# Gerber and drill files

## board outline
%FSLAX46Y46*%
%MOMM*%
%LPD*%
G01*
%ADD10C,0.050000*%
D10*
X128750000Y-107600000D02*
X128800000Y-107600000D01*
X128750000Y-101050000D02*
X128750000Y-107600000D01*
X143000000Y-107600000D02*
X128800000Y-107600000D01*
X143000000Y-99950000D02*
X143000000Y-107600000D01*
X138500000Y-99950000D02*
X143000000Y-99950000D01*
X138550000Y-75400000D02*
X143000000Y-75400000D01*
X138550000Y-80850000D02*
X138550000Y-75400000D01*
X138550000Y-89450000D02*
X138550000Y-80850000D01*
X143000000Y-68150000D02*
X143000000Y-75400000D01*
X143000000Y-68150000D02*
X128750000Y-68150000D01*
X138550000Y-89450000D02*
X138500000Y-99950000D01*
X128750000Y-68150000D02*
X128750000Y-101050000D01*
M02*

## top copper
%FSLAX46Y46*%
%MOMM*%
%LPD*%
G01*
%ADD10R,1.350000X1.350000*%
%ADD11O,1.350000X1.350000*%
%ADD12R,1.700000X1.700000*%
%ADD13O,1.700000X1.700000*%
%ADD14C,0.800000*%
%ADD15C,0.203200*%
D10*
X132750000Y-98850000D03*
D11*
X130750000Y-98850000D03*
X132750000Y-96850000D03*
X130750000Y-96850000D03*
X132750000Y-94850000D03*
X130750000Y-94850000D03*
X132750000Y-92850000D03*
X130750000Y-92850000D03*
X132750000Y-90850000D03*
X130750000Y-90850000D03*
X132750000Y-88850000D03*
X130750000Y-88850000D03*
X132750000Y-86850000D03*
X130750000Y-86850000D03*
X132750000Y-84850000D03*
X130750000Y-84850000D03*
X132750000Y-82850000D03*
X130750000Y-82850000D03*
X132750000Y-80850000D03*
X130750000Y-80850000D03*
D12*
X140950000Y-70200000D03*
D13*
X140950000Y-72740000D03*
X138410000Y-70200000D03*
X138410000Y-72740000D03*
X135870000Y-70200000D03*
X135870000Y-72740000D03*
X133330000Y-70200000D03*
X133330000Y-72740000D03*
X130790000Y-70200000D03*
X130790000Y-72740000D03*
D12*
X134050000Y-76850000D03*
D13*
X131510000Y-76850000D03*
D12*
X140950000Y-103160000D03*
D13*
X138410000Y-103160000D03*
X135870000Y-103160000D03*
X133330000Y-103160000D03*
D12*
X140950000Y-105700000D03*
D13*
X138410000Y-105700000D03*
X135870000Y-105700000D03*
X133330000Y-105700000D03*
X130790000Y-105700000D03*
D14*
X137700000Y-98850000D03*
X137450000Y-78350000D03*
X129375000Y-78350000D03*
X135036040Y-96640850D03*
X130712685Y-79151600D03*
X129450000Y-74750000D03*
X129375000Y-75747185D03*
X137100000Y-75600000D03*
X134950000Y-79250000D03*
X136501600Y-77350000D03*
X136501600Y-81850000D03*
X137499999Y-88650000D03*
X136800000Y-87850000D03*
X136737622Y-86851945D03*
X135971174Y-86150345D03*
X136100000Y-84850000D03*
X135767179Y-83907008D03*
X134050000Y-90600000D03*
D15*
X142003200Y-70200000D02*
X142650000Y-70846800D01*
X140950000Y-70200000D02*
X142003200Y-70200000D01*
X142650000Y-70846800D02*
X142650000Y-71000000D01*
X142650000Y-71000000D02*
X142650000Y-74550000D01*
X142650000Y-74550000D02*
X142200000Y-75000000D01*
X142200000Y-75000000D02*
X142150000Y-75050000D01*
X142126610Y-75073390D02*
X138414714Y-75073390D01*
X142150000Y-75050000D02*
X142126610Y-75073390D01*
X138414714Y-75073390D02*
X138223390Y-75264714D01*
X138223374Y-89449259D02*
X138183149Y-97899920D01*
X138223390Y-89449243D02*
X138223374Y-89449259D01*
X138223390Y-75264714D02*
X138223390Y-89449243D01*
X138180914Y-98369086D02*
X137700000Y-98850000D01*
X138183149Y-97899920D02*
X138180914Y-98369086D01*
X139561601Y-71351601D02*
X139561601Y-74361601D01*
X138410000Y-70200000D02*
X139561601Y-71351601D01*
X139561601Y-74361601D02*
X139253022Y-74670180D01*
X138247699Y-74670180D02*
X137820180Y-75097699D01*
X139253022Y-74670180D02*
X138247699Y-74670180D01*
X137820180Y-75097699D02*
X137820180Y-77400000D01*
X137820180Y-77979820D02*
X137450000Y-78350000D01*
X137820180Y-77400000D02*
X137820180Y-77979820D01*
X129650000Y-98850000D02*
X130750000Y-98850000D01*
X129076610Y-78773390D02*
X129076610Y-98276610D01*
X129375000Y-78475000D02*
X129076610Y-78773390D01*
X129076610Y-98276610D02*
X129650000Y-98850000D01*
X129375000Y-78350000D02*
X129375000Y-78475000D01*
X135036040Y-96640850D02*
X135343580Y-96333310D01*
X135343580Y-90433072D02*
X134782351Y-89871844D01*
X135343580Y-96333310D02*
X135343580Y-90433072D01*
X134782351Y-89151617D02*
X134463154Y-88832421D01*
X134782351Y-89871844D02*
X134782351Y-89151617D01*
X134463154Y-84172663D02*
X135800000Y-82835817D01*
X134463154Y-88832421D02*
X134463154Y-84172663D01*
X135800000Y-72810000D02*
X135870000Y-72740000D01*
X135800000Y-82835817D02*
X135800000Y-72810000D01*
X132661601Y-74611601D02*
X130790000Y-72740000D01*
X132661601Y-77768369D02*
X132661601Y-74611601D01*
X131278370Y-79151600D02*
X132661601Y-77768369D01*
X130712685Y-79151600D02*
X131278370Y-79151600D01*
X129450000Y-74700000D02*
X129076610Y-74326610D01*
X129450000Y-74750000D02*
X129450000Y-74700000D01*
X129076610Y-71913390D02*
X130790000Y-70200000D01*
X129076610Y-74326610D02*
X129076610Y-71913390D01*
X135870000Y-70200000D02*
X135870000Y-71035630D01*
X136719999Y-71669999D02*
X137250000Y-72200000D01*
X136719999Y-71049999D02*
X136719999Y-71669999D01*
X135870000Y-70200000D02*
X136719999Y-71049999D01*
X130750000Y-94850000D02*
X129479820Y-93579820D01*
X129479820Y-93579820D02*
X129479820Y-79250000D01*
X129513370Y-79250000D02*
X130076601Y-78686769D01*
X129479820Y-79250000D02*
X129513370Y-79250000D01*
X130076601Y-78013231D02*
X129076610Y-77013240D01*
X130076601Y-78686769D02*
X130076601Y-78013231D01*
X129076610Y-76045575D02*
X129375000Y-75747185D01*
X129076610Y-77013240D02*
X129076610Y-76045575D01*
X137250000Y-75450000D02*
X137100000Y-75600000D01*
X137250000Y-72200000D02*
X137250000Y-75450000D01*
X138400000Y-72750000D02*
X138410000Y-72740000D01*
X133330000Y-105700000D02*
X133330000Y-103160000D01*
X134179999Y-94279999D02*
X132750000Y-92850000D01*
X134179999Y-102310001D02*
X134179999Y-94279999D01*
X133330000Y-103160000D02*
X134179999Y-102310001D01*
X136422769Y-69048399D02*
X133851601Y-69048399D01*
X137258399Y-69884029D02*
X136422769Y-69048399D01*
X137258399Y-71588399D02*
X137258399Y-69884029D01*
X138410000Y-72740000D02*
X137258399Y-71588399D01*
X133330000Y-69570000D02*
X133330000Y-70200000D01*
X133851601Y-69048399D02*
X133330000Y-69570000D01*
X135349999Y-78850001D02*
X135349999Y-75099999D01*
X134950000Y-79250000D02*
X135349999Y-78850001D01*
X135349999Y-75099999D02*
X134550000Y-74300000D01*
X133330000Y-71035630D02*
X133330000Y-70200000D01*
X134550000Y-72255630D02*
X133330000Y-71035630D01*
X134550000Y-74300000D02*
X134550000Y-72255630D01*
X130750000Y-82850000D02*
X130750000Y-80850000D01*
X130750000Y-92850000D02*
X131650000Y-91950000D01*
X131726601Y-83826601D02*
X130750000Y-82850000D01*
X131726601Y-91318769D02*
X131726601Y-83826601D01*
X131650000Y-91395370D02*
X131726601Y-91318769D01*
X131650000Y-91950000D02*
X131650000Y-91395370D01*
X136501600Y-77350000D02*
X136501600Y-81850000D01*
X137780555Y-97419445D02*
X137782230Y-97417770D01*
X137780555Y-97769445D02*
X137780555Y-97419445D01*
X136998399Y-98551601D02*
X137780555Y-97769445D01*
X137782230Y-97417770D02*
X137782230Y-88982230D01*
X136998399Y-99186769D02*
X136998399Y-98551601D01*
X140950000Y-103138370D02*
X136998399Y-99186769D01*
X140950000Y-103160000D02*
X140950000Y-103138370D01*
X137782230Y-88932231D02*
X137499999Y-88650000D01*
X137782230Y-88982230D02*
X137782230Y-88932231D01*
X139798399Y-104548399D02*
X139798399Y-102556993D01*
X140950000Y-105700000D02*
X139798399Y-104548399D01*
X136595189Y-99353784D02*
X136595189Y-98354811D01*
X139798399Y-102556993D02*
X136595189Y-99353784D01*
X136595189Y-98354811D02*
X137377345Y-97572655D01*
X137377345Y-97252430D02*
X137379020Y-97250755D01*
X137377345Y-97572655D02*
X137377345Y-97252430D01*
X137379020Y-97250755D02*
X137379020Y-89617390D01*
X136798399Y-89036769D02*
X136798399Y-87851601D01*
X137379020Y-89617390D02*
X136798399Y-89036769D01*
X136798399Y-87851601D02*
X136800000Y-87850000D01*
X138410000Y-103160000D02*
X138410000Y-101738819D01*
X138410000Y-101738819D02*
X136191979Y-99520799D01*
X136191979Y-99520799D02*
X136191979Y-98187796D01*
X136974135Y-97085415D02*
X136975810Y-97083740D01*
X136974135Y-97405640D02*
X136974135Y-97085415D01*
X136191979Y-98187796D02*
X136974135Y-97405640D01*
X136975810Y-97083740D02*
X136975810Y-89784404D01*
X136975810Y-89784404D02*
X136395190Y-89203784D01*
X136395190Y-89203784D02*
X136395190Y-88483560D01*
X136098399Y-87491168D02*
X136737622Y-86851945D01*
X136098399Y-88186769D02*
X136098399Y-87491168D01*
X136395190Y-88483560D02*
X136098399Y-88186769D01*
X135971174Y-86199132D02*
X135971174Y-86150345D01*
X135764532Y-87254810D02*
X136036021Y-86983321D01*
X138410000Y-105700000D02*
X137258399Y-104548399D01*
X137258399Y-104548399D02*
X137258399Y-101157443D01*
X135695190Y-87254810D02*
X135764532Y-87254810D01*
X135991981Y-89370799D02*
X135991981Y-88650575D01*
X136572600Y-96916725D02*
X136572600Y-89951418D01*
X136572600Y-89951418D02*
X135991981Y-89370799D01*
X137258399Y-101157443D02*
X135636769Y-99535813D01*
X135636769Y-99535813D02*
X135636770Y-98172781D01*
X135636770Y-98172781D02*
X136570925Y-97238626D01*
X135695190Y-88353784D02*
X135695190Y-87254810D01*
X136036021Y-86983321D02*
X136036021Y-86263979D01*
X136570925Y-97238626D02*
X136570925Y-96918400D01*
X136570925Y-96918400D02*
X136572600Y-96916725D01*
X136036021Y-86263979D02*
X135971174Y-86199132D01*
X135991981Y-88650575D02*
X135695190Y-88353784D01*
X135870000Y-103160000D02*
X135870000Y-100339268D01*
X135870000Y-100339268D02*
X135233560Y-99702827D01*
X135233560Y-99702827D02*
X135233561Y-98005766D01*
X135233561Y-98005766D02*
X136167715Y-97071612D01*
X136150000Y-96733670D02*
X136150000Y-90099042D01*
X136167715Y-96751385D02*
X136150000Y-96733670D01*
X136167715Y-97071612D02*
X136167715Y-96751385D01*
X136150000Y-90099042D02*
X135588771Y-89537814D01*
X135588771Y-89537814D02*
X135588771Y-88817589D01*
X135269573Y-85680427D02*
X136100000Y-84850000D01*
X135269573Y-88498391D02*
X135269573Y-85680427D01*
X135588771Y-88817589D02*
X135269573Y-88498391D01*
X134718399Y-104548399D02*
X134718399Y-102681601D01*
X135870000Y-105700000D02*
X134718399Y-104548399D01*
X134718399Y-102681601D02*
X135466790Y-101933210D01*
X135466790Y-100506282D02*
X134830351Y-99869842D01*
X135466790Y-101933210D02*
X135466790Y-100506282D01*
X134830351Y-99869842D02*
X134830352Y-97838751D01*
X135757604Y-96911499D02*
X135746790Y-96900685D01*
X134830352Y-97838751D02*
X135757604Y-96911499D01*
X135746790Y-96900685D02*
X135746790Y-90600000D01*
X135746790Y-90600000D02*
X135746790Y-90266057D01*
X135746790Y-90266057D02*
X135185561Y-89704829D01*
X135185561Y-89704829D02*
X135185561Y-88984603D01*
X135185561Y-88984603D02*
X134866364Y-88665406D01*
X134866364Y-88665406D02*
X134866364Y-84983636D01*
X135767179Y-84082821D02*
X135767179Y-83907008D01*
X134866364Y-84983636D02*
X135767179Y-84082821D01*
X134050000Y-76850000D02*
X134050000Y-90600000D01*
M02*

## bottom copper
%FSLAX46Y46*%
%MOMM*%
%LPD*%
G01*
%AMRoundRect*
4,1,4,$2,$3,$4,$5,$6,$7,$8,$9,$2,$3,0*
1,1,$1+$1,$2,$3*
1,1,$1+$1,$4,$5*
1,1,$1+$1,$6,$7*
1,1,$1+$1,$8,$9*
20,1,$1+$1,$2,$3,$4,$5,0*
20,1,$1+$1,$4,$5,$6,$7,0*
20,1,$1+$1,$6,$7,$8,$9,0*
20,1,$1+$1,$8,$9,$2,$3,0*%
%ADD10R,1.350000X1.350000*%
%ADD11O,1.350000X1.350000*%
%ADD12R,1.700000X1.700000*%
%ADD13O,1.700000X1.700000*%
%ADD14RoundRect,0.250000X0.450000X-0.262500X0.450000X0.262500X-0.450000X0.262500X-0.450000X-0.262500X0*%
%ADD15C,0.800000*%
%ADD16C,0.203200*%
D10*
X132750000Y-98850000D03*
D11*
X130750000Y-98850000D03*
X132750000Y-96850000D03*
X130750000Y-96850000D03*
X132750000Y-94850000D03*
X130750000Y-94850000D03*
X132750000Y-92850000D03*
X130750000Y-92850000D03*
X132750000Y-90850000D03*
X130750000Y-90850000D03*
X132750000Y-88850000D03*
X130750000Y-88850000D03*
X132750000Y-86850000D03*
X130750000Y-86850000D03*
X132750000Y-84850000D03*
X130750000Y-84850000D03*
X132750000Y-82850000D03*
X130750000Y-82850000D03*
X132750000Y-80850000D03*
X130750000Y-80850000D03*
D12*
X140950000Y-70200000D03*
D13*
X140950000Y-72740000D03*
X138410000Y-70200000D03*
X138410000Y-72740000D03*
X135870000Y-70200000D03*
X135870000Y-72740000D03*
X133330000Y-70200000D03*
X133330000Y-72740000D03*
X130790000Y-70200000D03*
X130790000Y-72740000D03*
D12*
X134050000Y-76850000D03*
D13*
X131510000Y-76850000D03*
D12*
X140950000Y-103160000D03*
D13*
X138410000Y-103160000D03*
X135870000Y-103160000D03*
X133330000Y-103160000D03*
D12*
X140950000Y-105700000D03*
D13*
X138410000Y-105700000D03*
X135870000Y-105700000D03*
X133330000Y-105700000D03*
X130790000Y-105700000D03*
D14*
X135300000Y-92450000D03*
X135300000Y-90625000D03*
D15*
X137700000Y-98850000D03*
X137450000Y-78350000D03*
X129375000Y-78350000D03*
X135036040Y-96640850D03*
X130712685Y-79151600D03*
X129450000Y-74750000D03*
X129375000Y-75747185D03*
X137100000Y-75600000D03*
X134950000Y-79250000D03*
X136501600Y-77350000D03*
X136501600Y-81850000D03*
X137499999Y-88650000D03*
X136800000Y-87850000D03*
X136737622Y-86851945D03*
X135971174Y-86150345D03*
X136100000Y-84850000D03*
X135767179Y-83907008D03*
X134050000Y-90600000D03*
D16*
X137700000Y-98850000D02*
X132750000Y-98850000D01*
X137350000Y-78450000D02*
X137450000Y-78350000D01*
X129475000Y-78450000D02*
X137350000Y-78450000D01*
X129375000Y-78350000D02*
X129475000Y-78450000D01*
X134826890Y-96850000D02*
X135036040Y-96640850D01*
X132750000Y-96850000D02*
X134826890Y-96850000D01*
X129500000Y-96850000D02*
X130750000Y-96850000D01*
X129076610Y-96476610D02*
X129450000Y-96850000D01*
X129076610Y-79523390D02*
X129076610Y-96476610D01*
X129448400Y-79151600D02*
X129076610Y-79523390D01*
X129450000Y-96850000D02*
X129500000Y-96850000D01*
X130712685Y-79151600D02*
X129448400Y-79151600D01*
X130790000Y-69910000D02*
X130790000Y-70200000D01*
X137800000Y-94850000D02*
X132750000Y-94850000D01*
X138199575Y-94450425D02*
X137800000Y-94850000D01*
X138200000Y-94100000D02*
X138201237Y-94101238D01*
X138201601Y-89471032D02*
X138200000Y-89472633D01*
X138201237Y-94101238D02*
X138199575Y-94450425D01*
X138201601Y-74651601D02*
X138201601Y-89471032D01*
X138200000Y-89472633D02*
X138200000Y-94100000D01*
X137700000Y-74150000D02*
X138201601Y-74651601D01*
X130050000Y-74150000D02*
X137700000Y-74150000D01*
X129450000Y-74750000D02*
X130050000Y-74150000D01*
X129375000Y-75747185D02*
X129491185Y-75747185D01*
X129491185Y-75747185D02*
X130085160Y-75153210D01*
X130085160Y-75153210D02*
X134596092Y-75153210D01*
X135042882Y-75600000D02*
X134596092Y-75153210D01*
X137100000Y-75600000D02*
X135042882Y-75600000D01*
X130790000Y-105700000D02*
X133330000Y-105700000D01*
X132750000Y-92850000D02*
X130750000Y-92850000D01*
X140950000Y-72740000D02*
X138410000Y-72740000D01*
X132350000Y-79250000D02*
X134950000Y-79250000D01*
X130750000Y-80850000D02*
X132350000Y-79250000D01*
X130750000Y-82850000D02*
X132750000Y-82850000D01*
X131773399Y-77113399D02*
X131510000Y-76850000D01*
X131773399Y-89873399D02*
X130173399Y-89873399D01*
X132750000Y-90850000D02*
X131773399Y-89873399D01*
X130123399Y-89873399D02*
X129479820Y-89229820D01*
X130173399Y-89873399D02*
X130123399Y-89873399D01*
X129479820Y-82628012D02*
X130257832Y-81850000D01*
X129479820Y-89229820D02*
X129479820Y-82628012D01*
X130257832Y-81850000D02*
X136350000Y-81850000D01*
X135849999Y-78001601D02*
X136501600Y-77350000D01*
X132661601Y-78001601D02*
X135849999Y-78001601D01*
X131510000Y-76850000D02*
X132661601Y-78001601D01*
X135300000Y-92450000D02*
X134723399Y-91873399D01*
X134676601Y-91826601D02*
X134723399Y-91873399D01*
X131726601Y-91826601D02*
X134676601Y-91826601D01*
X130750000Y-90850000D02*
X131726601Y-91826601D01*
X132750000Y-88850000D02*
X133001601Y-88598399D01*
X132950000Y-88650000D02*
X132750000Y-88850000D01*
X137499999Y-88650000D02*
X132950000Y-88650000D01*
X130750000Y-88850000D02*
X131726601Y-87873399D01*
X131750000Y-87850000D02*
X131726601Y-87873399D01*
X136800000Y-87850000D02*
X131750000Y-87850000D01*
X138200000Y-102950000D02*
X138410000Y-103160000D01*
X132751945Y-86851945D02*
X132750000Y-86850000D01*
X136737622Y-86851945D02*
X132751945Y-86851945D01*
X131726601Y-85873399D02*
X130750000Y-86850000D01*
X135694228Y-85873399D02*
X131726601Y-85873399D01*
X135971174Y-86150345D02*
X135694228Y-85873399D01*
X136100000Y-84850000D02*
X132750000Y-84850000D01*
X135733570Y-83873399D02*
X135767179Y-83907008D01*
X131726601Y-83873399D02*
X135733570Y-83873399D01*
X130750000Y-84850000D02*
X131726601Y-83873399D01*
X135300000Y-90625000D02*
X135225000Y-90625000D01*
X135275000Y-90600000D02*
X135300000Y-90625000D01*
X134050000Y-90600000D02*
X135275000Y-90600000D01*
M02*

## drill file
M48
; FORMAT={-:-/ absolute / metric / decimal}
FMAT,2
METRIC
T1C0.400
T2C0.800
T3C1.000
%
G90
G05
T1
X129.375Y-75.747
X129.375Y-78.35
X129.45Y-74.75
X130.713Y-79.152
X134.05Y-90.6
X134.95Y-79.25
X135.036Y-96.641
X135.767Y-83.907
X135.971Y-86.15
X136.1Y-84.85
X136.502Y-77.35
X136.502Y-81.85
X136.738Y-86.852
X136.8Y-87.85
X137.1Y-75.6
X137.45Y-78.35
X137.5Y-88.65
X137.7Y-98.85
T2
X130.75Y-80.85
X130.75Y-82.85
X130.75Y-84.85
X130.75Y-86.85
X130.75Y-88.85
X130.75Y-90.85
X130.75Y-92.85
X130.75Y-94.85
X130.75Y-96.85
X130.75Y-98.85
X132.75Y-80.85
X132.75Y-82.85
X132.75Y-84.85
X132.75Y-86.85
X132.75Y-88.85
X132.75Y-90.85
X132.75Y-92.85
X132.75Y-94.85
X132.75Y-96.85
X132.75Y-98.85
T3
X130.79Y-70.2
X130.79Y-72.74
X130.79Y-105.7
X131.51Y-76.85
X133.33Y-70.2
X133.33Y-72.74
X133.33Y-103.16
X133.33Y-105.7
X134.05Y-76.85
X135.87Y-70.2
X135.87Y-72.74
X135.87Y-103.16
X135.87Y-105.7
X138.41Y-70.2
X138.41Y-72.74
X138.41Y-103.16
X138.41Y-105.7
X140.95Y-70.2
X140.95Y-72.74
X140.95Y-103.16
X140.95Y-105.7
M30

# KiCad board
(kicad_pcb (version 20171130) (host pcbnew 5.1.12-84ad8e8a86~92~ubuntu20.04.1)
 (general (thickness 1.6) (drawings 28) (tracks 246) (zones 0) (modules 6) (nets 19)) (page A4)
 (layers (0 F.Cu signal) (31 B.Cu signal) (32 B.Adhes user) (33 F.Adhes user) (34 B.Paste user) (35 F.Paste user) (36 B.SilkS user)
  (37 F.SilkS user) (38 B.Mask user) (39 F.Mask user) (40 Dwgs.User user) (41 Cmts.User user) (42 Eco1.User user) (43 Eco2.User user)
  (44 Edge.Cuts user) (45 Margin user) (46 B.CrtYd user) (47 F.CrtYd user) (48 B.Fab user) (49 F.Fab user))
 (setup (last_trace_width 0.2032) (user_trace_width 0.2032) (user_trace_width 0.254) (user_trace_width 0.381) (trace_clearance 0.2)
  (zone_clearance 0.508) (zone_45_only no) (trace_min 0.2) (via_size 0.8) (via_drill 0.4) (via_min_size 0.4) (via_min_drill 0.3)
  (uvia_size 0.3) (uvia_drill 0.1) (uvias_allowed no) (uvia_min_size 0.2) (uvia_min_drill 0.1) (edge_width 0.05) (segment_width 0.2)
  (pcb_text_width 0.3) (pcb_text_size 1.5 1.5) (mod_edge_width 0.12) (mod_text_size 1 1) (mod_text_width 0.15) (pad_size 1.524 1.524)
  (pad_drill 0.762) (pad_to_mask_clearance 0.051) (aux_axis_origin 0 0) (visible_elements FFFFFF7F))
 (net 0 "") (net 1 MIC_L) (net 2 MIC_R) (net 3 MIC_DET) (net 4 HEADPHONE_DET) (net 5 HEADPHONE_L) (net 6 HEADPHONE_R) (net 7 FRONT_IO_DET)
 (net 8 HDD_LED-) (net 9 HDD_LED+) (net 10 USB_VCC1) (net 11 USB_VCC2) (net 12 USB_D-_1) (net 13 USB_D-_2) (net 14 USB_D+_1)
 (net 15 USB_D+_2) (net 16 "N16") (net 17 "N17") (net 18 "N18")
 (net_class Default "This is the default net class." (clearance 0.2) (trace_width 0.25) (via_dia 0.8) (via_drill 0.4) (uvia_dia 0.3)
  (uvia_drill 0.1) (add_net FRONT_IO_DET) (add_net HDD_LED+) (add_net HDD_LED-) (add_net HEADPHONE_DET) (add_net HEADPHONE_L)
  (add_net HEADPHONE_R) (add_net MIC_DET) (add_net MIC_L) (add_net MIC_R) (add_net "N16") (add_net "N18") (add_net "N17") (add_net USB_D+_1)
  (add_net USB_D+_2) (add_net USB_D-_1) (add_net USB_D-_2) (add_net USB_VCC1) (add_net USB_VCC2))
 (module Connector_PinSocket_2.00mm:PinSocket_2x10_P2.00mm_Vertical (layer B.Cu) (at 132.75 98.85)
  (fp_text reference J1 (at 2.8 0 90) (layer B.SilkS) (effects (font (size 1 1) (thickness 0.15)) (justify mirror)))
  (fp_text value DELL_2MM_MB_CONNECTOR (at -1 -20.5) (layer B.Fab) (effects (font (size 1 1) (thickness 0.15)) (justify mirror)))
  (pad 1 thru_hole rect (at 0 0) (size 1.35 1.35) (drill 0.8) (layers *.Cu *.Mask) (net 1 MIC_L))
  (pad 2 thru_hole oval (at -2 0) (size 1.35 1.35) (drill 0.8) (layers *.Cu *.Mask) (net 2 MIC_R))
  (pad 3 thru_hole oval (at 0 -2) (size 1.35 1.35) (drill 0.8) (layers *.Cu *.Mask) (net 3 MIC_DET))
  (pad 4 thru_hole oval (at -2 -2) (size 1.35 1.35) (drill 0.8) (layers *.Cu *.Mask) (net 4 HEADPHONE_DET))
  (pad 5 thru_hole oval (at 0 -4) (size 1.35 1.35) (drill 0.8) (layers *.Cu *.Mask) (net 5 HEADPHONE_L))
  (pad 6 thru_hole oval (at -2 -4) (size 1.35 1.35) (drill 0.8) (layers *.Cu *.Mask) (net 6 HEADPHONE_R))
  (pad 7 thru_hole oval (at 0 -6) (size 1.35 1.35) (drill 0.8) (layers *.Cu *.Mask) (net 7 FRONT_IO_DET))
  (pad 8 thru_hole oval (at -2 -6) (size 1.35 1.35) (drill 0.8) (layers *.Cu *.Mask) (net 7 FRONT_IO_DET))
  (pad 9 thru_hole oval (at 0 -8) (size 1.35 1.35) (drill 0.8) (layers *.Cu *.Mask) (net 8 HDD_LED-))
  (pad 10 thru_hole oval (at -2 -8) (size 1.35 1.35) (drill 0.8) (layers *.Cu *.Mask) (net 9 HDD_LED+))
  (pad 11 thru_hole oval (at 0 -10) (size 1.35 1.35) (drill 0.8) (layers *.Cu *.Mask) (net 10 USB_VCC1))
  (pad 12 thru_hole oval (at -2 -10) (size 1.35 1.35) (drill 0.8) (layers *.Cu *.Mask) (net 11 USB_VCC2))
  (pad 13 thru_hole oval (at 0 -12) (size 1.35 1.35) (drill 0.8) (layers *.Cu *.Mask) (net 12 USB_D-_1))
  (pad 14 thru_hole oval (at -2 -12) (size 1.35 1.35) (drill 0.8) (layers *.Cu *.Mask) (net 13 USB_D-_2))
  (pad 15 thru_hole oval (at 0 -14) (size 1.35 1.35) (drill 0.8) (layers *.Cu *.Mask) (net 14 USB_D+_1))
  (pad 16 thru_hole oval (at -2 -14) (size 1.35 1.35) (drill 0.8) (layers *.Cu *.Mask) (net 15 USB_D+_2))
  (pad 17 thru_hole oval (at 0 -16) (size 1.35 1.35) (drill 0.8) (layers *.Cu *.Mask) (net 7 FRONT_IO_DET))
  (pad 18 thru_hole oval (at -2 -16) (size 1.35 1.35) (drill 0.8) (layers *.Cu *.Mask) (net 7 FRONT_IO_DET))
  (pad 19 thru_hole oval (at 0 -18) (size 1.35 1.35) (drill 0.8) (layers *.Cu *.Mask) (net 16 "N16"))
  (pad 20 thru_hole oval (at -2 -18) (size 1.35 1.35) (drill 0.8) (layers *.Cu *.Mask) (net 7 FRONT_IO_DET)))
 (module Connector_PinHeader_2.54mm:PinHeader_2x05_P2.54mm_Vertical (layer F.Cu) (at 140.95 70.2 270)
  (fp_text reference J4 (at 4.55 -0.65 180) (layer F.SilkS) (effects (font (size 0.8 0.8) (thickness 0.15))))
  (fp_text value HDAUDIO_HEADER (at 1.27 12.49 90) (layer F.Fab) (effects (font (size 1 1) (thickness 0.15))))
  (pad 1 thru_hole rect (at 0 0 270) (size 1.7 1.7) (drill 1) (layers *.Cu *.Mask) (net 1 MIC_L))
  (pad 2 thru_hole oval (at 2.54 0 270) (size 1.7 1.7) (drill 1) (layers *.Cu *.Mask) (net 7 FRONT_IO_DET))
  (pad 3 thru_hole oval (at 0 2.54 270) (size 1.7 1.7) (drill 1) (layers *.Cu *.Mask) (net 2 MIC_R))
  (pad 4 thru_hole oval (at 2.54 2.54 270) (size 1.7 1.7) (drill 1) (layers *.Cu *.Mask) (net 7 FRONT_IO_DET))
  (pad 5 thru_hole oval (at 0 5.08 270) (size 1.7 1.7) (drill 1) (layers *.Cu *.Mask) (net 6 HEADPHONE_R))
  (pad 6 thru_hole oval (at 2.54 5.08 270) (size 1.7 1.7) (drill 1) (layers *.Cu *.Mask) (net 3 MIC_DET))
  (pad 7 thru_hole oval (at 0 7.62 270) (size 1.7 1.7) (drill 1) (layers *.Cu *.Mask) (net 7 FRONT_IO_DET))
  (pad 8 thru_hole oval (at 2.54 7.62 270) (size 1.7 1.7) (drill 1) (layers *.Cu *.Mask) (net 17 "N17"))
  (pad 9 thru_hole oval (at 0 10.16 270) (size 1.7 1.7) (drill 1) (layers *.Cu *.Mask) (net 5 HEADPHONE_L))
  (pad 10 thru_hole oval (at 2.54 10.16 270) (size 1.7 1.7) (drill 1) (layers *.Cu *.Mask) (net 4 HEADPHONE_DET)))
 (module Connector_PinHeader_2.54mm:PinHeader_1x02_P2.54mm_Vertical (layer F.Cu) (at 134.05 76.85 270)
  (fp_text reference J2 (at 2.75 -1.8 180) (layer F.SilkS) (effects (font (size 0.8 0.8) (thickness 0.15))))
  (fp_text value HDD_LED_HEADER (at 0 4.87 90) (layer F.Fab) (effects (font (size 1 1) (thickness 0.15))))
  (pad 1 thru_hole rect (at 0 0 270) (size 1.7 1.7) (drill 1) (layers *.Cu *.Mask) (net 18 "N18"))
  (pad 2 thru_hole oval (at 0 2.54 270) (size 1.7 1.7) (drill 1) (layers *.Cu *.Mask) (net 8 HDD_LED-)))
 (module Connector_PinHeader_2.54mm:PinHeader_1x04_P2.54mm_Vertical (layer F.Cu) (at 140.95 103.16 270)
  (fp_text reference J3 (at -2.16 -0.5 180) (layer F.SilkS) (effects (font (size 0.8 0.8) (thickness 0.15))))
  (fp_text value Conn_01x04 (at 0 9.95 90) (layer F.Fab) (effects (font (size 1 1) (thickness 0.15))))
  (pad 1 thru_hole rect (at 0 0 270) (size 1.7 1.7) (drill 1) (layers *.Cu *.Mask) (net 10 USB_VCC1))
  (pad 2 thru_hole oval (at 0 2.54 270) (size 1.7 1.7) (drill 1) (layers *.Cu *.Mask) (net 12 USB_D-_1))
  (pad 3 thru_hole oval (at 0 5.08 270) (size 1.7 1.7) (drill 1) (layers *.Cu *.Mask) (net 14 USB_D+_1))
  (pad 4 thru_hole oval (at 0 7.62 270) (size 1.7 1.7) (drill 1) (layers *.Cu *.Mask) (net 7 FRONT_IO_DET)))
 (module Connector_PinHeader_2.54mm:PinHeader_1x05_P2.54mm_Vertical (layer F.Cu) (at 140.95 105.7 270)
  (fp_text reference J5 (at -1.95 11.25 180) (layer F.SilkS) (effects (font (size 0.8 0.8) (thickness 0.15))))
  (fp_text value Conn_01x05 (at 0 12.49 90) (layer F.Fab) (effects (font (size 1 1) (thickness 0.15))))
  (pad 1 thru_hole rect (at 0 0 270) (size 1.7 1.7) (drill 1) (layers *.Cu *.Mask) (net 11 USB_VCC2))
  (pad 2 thru_hole oval (at 0 2.54 270) (size 1.7 1.7) (drill 1) (layers *.Cu *.Mask) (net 13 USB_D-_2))
  (pad 3 thru_hole oval (at 0 5.08 270) (size 1.7 1.7) (drill 1) (layers *.Cu *.Mask) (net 15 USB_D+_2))
  (pad 4 thru_hole oval (at 0 7.62 270) (size 1.7 1.7) (drill 1) (layers *.Cu *.Mask) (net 7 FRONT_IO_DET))
  (pad 5 thru_hole oval (at 0 10.16 270) (size 1.7 1.7) (drill 1) (layers *.Cu *.Mask) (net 7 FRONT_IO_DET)))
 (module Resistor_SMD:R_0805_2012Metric (layer B.Cu) (at 135.3 91.5375 90)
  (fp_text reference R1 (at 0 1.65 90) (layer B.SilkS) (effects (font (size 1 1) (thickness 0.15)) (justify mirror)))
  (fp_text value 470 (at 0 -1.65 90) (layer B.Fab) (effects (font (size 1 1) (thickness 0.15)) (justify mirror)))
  (pad 1 smd roundrect (at -0.9125 0 90) (size 1.025 1.4) (layers B.Cu B.Paste B.Mask) (roundrect_rratio 0.243902) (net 9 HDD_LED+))
  (pad 2 smd roundrect (at 0.9125 0 90) (size 1.025 1.4) (layers B.Cu B.Paste B.Mask) (roundrect_rratio 0.243902) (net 18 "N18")))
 (gr_line (start 128.75 107.6) (end 128.8 107.6) (layer Edge.Cuts) (width 0.05))
 (gr_line (start 128.75 101.05) (end 128.75 107.6) (layer Edge.Cuts) (width 0.05))
 (gr_line (start 143 107.6) (end 128.8 107.6) (layer Edge.Cuts) (width 0.05))
 (gr_line (start 143 99.95) (end 143 107.6) (layer Edge.Cuts) (width 0.05))
 (gr_line (start 138.5 99.95) (end 143 99.95) (layer Edge.Cuts) (width 0.05))
 (gr_line (start 138.55 75.4) (end 143 75.4) (layer Edge.Cuts) (width 0.05))
 (gr_line (start 138.55 80.85) (end 138.55 75.4) (layer Edge.Cuts) (width 0.05))
 (gr_line (start 138.55 89.45) (end 138.55 80.85) (layer Edge.Cuts) (width 0.05))
 (gr_line (start 143 68.15) (end 143 75.4) (layer Edge.Cuts) (width 0.05))
 (gr_line (start 143 68.15) (end 128.75 68.15) (layer Edge.Cuts) (width 0.05))
 (gr_line (start 138.55 89.45) (end 138.5 99.95) (layer Edge.Cuts) (width 0.05))
 (gr_line (start 128.75 68.15) (end 128.75 101.05) (layer Edge.Cuts) (width 0.05))
 (segment (start 142.0032 70.2) (end 142.65 70.8468) (width 0.2032) (layer F.Cu) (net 1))
 (segment (start 140.95 70.2) (end 142.0032 70.2) (width 0.2032) (layer F.Cu) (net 1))
 (segment (start 142.65 70.8468) (end 142.65 71) (width 0.2032) (layer F.Cu) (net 1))
 (segment (start 142.65 71) (end 142.65 74.55) (width 0.2032) (layer F.Cu) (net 1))
 (segment (start 142.65 74.55) (end 142.2 75) (width 0.2032) (layer F.Cu) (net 1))
 (segment (start 142.2 75) (end 142.15 75.05) (width 0.2032) (layer F.Cu) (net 1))
 (segment (start 142.12661 75.07339) (end 138.414714 75.07339) (width 0.2032) (layer F.Cu) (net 1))
 (segment (start 142.15 75.05) (end 142.12661 75.07339) (width 0.2032) (layer F.Cu) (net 1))
 (segment (start 138.414714 75.07339) (end 138.22339 75.264714) (width 0.2032) (layer F.Cu) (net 1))
 (segment (start 138.223374 89.449259) (end 138.183149 97.89992) (width 0.2032) (layer F.Cu) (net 1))
 (segment (start 138.22339 89.449243) (end 138.223374 89.449259) (width 0.2032) (layer F.Cu) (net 1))
 (segment (start 138.22339 75.264714) (end 138.22339 89.449243) (width 0.2032) (layer F.Cu) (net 1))
 (via (at 137.7 98.85) (size 0.8) (drill 0.4) (layers F.Cu B.Cu) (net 1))
 (segment (start 138.180914 98.369086) (end 137.7 98.85) (width 0.2032) (layer F.Cu) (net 1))
 (segment (start 138.183149 97.89992) (end 138.180914 98.369086) (width 0.2032) (layer F.Cu) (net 1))
 (segment (start 137.7 98.85) (end 132.75 98.85) (width 0.2032) (layer B.Cu) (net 1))
 (segment (start 139.561601 71.351601) (end 139.561601 74.361601) (width 0.2032) (layer F.Cu) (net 2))
 (segment (start 138.41 70.2) (end 139.561601 71.351601) (width 0.2032) (layer F.Cu) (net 2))
 (segment (start 139.561601 74.361601) (end 139.253022 74.67018) (width 0.2032) (layer F.Cu) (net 2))
 (segment (start 138.247699 74.67018) (end 137.82018 75.097699) (width 0.2032) (layer F.Cu) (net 2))
 (segment (start 139.253022 74.67018) (end 138.247699 74.67018) (width 0.2032) (layer F.Cu) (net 2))
 (segment (start 137.82018 75.097699) (end 137.82018 77.4) (width 0.2032) (layer F.Cu) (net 2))
 (via (at 137.45 78.35) (size 0.8) (drill 0.4) (layers F.Cu B.Cu) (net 2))
 (segment (start 137.82018 77.97982) (end 137.45 78.35) (width 0.2032) (layer F.Cu) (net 2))
 (segment (start 137.82018 77.4) (end 137.82018 77.97982) (width 0.2032) (layer F.Cu) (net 2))
 (via (at 129.375 78.35) (size 0.8) (drill 0.4) (layers F.Cu B.Cu) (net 2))
 (segment (start 129.65 98.85) (end 130.75 98.85) (width 0.2032) (layer F.Cu) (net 2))
 (segment (start 129.07661 78.77339) (end 129.07661 98.27661) (width 0.2032) (layer F.Cu) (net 2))
 (segment (start 129.375 78.475) (end 129.07661 78.77339) (width 0.2032) (layer F.Cu) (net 2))
 (segment (start 129.07661 98.27661) (end 129.65 98.85) (width 0.2032) (layer F.Cu) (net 2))
 (segment (start 129.375 78.35) (end 129.375 78.475) (width 0.2032) (layer F.Cu) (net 2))
 (segment (start 137.35 78.45) (end 137.45 78.35) (width 0.2032) (layer B.Cu) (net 2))
 (segment (start 129.475 78.45) (end 137.35 78.45) (width 0.2032) (layer B.Cu) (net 2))
 (segment (start 129.375 78.35) (end 129.475 78.45) (width 0.2032) (layer B.Cu) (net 2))
 (via (at 135.03604 96.64085) (size 0.8) (drill 0.4) (layers F.Cu B.Cu) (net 3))
 (segment (start 134.82689 96.85) (end 135.03604 96.64085) (width 0.2032) (layer B.Cu) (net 3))
 (segment (start 132.75 96.85) (end 134.82689 96.85) (width 0.2032) (layer B.Cu) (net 3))
 (segment (start 135.03604 96.64085) (end 135.34358 96.33331) (width 0.2032) (layer F.Cu) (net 3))
 (segment (start 135.34358 90.433072) (end 134.782351 89.871844) (width 0.2032) (layer F.Cu) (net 3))
 (segment (start 135.34358 96.33331) (end 135.34358 90.433072) (width 0.2032) (layer F.Cu) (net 3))
 (segment (start 134.782351 89.151617) (end 134.463154 88.832421) (width 0.2032) (layer F.Cu) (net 3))
 (segment (start 134.782351 89.871844) (end 134.782351 89.151617) (width 0.2032) (layer F.Cu) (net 3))
 (segment (start 134.463154 84.172663) (end 135.8 82.835817) (width 0.2032) (layer F.Cu) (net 3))
 (segment (start 134.463154 88.832421) (end 134.463154 84.172663) (width 0.2032) (layer F.Cu) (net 3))
 (segment (start 135.8 72.81) (end 135.87 72.74) (width 0.2032) (layer F.Cu) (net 3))
 (segment (start 135.8 82.835817) (end 135.8 72.81) (width 0.2032) (layer F.Cu) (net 3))
 (via (at 130.712685 79.1516) (size 0.8) (drill 0.4) (layers F.Cu B.Cu) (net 4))
 (segment (start 132.661601 74.611601) (end 130.79 72.74) (width 0.2032) (layer F.Cu) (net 4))
 (segment (start 132.661601 77.768369) (end 132.661601 74.611601) (width 0.2032) (layer F.Cu) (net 4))
 (segment (start 131.27837 79.1516) (end 132.661601 77.768369) (width 0.2032) (layer F.Cu) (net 4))
 (segment (start 130.712685 79.1516) (end 131.27837 79.1516) (width 0.2032) (layer F.Cu) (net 4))
 (segment (start 129.5 96.85) (end 130.75 96.85) (width 0.2032) (layer B.Cu) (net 4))
 (segment (start 129.07661 96.47661) (end 129.45 96.85) (width 0.2032) (layer B.Cu) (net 4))
 (segment (start 129.07661 79.52339) (end 129.07661 96.47661) (width 0.2032) (layer B.Cu) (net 4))
 (segment (start 129.4484 79.1516) (end 129.07661 79.52339) (width 0.2032) (layer B.Cu) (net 4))
 (segment (start 129.45 96.85) (end 129.5 96.85) (width 0.2032) (layer B.Cu) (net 4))
 (segment (start 130.712685 79.1516) (end 129.4484 79.1516) (width 0.2032) (layer B.Cu) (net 4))
 (segment (start 130.79 69.91) (end 130.79 70.2) (width 0.2032) (layer B.Cu) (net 5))
 (via (at 129.45 74.75) (size 0.8) (drill 0.4) (layers F.Cu B.Cu) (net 5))
 (segment (start 129.45 74.7) (end 129.07661 74.32661) (width 0.2032) (layer F.Cu) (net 5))
 (segment (start 129.45 74.75) (end 129.45 74.7) (width 0.2032) (layer F.Cu) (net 5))
 (segment (start 129.07661 71.91339) (end 130.79 70.2) (width 0.2032) (layer F.Cu) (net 5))
 (segment (start 129.07661 74.32661) (end 129.07661 71.91339) (width 0.2032) (layer F.Cu) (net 5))
 (segment (start 137.8 94.85) (end 132.75 94.85) (width 0.2032) (layer B.Cu) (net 5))
 (segment (start 138.199575 94.450425) (end 137.8 94.85) (width 0.2032) (layer B.Cu) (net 5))
 (segment (start 138.2 94.1) (end 138.201237 94.101238) (width 0.2032) (layer B.Cu) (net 5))
 (segment (start 138.201601 89.471032) (end 138.2 89.472633) (width 0.2032) (layer B.Cu) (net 5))
 (segment (start 138.201237 94.101238) (end 138.199575 94.450425) (width 0.2032) (layer B.Cu) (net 5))
 (segment (start 138.201601 74.651601) (end 138.201601 89.471032) (width 0.2032) (layer B.Cu) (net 5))
 (segment (start 138.2 89.472633) (end 138.2 94.1) (width 0.2032) (layer B.Cu) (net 5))
 (segment (start 137.7 74.15) (end 138.201601 74.651601) (width 0.2032) (layer B.Cu) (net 5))
 (segment (start 130.05 74.15) (end 137.7 74.15) (width 0.2032) (layer B.Cu) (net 5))
 (segment (start 129.45 74.75) (end 130.05 74.15) (width 0.2032) (layer B.Cu) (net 5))
 (segment (start 135.87 70.2) (end 135.87 71.03563) (width 0.2032) (layer F.Cu) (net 6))
 (segment (start 136.719999 71.669999) (end 137.25 72.2) (width 0.2032) (layer F.Cu) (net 6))
 (segment (start 136.719999 71.049999) (end 136.719999 71.669999) (width 0.2032) (layer F.Cu) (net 6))
 (segment (start 135.87 70.2) (end 136.719999 71.049999) (width 0.2032) (layer F.Cu) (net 6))
 (segment (start 130.75 94.85) (end 129.47982 93.57982) (width 0.2032) (layer F.Cu) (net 6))
 (segment (start 129.47982 93.57982) (end 129.47982 79.25) (width 0.2032) (layer F.Cu) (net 6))
 (segment (start 129.51337 79.25) (end 130.076601 78.686769) (width 0.2032) (layer F.Cu) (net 6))
 (segment (start 129.47982 79.25) (end 129.51337 79.25) (width 0.2032) (layer F.Cu) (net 6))
 (segment (start 130.076601 78.013231) (end 129.07661 77.01324) (width 0.2032) (layer F.Cu) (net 6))
 (segment (start 130.076601 78.686769) (end 130.076601 78.013231) (width 0.2032) (layer F.Cu) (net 6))
 (via (at 129.375 75.747185) (size 0.8) (drill 0.4) (layers F.Cu B.Cu) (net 6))
 (segment (start 129.07661 76.045575) (end 129.375 75.747185) (width 0.2032) (layer F.Cu) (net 6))
 (segment (start 129.07661 77.01324) (end 129.07661 76.045575) (width 0.2032) (layer F.Cu) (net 6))
 (segment (start 129.375 75.747185) (end 129.491185 75.747185) (width 0.2032) (layer B.Cu) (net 6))
 (segment (start 129.491185 75.747185) (end 130.08516 75.15321) (width 0.2032) (layer B.Cu) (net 6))
 (segment (start 130.08516 75.15321) (end 134.596092 75.15321) (width 0.2032) (layer B.Cu) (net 6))
 (via (at 137.1 75.6) (size 0.8) (drill 0.4) (layers F.Cu B.Cu) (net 6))
 (segment (start 137.25 75.45) (end 137.1 75.6) (width 0.2032) (layer F.Cu) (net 6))
 (segment (start 137.25 72.2) (end 137.25 75.45) (width 0.2032) (layer F.Cu) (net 6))
 (segment (start 135.042882 75.6) (end 134.596092 75.15321) (width 0.2032) (layer B.Cu) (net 6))
 (segment (start 137.1 75.6) (end 135.042882 75.6) (width 0.2032) (layer B.Cu) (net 6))
 (segment (start 138.4 72.75) (end 138.41 72.74) (width 0.2032) (layer F.Cu) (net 7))
 (segment (start 130.79 105.7) (end 133.33 105.7) (width 0.2032) (layer B.Cu) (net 7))
 (segment (start 133.33 105.7) (end 133.33 103.16) (width 0.2032) (layer F.Cu) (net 7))
 (segment (start 134.179999 94.279999) (end 132.75 92.85) (width 0.2032) (layer F.Cu) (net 7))
 (segment (start 134.179999 102.310001) (end 134.179999 94.279999) (width 0.2032) (layer F.Cu) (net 7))
 (segment (start 133.33 103.16) (end 134.179999 102.310001) (width 0.2032) (layer F.Cu) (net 7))
 (segment (start 132.75 92.85) (end 130.75 92.85) (width 0.2032) (layer B.Cu) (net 7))
 (segment (start 140.95 72.74) (end 138.41 72.74) (width 0.2032) (layer B.Cu) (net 7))
 (segment (start 136.422769 69.048399) (end 133.851601 69.048399) (width 0.2032) (layer F.Cu) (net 7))
 (segment (start 137.258399 69.884029) (end 136.422769 69.048399) (width 0.2032) (layer F.Cu) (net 7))
 (segment (start 137.258399 71.588399) (end 137.258399 69.884029) (width 0.2032) (layer F.Cu) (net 7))
 (segment (start 138.41 72.74) (end 137.258399 71.588399) (width 0.2032) (layer F.Cu) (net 7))
 (segment (start 133.33 69.57) (end 133.33 70.2) (width 0.2032) (layer F.Cu) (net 7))
 (segment (start 133.851601 69.048399) (end 133.33 69.57) (width 0.2032) (layer F.Cu) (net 7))
 (segment (start 132.35 79.25) (end 134.95 79.25) (width 0.2032) (layer B.Cu) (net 7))
 (via (at 134.95 79.25) (size 0.8) (drill 0.4) (layers F.Cu B.Cu) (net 7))
 (segment (start 130.75 80.85) (end 132.35 79.25) (width 0.2032) (layer B.Cu) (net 7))
 (segment (start 135.349999 78.850001) (end 135.349999 75.099999) (width 0.2032) (layer F.Cu) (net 7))
 (segment (start 134.95 79.25) (end 135.349999 78.850001) (width 0.2032) (layer F.Cu) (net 7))
 (segment (start 135.349999 75.099999) (end 134.55 74.3) (width 0.2032) (layer F.Cu) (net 7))
 (segment (start 133.33 71.03563) (end 133.33 70.2) (width 0.2032) (layer F.Cu) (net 7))
 (segment (start 134.55 72.25563) (end 133.33 71.03563) (width 0.2032) (layer F.Cu) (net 7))
 (segment (start 134.55 74.3) (end 134.55 72.25563) (width 0.2032) (layer F.Cu) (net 7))
 (segment (start 130.75 82.85) (end 130.75 80.85) (width 0.2032) (layer F.Cu) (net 7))
 (segment (start 130.75 82.85) (end 132.75 82.85) (width 0.2032) (layer B.Cu) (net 7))
 (segment (start 130.75 92.85) (end 131.65 91.95) (width 0.2032) (layer F.Cu) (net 7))
 (segment (start 131.726601 83.826601) (end 130.75 82.85) (width 0.2032) (layer F.Cu) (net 7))
 (segment (start 131.726601 91.318769) (end 131.726601 83.826601) (width 0.2032) (layer F.Cu) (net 7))
 (segment (start 131.65 91.39537) (end 131.726601 91.318769) (width 0.2032) (layer F.Cu) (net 7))
 (segment (start 131.65 91.95) (end 131.65 91.39537) (width 0.2032) (layer F.Cu) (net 7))
 (segment (start 131.773399 77.113399) (end 131.51 76.85) (width 0.2032) (layer B.Cu) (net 8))
 (segment (start 131.773399 89.873399) (end 130.173399 89.873399) (width 0.2032) (layer B.Cu) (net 8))
 (segment (start 132.75 90.85) (end 131.773399 89.873399) (width 0.2032) (layer B.Cu) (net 8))
 (segment (start 130.123399 89.873399) (end 129.47982 89.22982) (width 0.2032) (layer B.Cu) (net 8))
 (segment (start 130.173399 89.873399) (end 130.123399 89.873399) (width 0.2032) (layer B.Cu) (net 8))
 (segment (start 129.47982 82.628012) (end 130.257832 81.85) (width 0.2032) (layer B.Cu) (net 8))
 (segment (start 129.47982 89.22982) (end 129.47982 82.628012) (width 0.2032) (layer B.Cu) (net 8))
 (segment (start 130.257832 81.85) (end 136.35 81.85) (width 0.2032) (layer B.Cu) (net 8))
 (via (at 136.5016 77.35) (size 0.8) (drill 0.4) (layers F.Cu B.Cu) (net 8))
 (segment (start 135.849999 78.001601) (end 136.5016 77.35) (width 0.2032) (layer B.Cu) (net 8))
 (segment (start 132.661601 78.001601) (end 135.849999 78.001601) (width 0.2032) (layer B.Cu) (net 8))
 (segment (start 131.51 76.85) (end 132.661601 78.001601) (width 0.2032) (layer B.Cu) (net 8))
 (via (at 136.5016 81.85) (size 0.8) (drill 0.4) (layers F.Cu B.Cu) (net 8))
 (segment (start 136.5016 77.35) (end 136.5016 81.85) (width 0.2032) (layer F.Cu) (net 8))
 (segment (start 135.3 92.45) (end 134.723399 91.873399) (width 0.2032) (layer B.Cu) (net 9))
 (segment (start 134.676601 91.826601) (end 134.723399 91.873399) (width 0.2032) (layer B.Cu) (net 9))
 (segment (start 131.726601 91.826601) (end 134.676601 91.826601) (width 0.2032) (layer B.Cu) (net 9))
 (segment (start 130.75 90.85) (end 131.726601 91.826601) (width 0.2032) (layer B.Cu) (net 9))
 (segment (start 132.75 88.85) (end 133.001601 88.598399) (width 0.2032) (layer B.Cu) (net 10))
 (segment (start 137.780555 97.419445) (end 137.78223 97.41777) (width 0.2032) (layer F.Cu) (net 10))
 (segment (start 137.780555 97.769445) (end 137.780555 97.419445) (width 0.2032) (layer F.Cu) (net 10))
 (segment (start 136.998399 98.551601) (end 137.780555 97.769445) (width 0.2032) (layer F.Cu) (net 10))
 (segment (start 137.78223 97.41777) (end 137.78223 88.98223) (width 0.2032) (layer F.Cu) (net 10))
 (segment (start 136.998399 99.186769) (end 136.998399 98.551601) (width 0.2032) (layer F.Cu) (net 10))
 (segment (start 140.95 103.13837) (end 136.998399 99.186769) (width 0.2032) (layer F.Cu) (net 10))
 (segment (start 140.95 103.16) (end 140.95 103.13837) (width 0.2032) (layer F.Cu) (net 10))
 (via (at 137.499999 88.65) (size 0.8) (drill 0.4) (layers F.Cu B.Cu) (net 10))
 (segment (start 137.78223 88.932231) (end 137.499999 88.65) (width 0.2032) (layer F.Cu) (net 10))
 (segment (start 137.78223 88.98223) (end 137.78223 88.932231) (width 0.2032) (layer F.Cu) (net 10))
 (segment (start 132.95 88.65) (end 132.75 88.85) (width 0.2032) (layer B.Cu) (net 10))
 (segment (start 137.499999 88.65) (end 132.95 88.65) (width 0.2032) (layer B.Cu) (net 10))
 (segment (start 130.75 88.85) (end 131.726601 87.873399) (width 0.2032) (layer B.Cu) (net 11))
 (segment (start 139.798399 104.548399) (end 139.798399 102.556993) (width 0.2032) (layer F.Cu) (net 11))
 (segment (start 140.95 105.7) (end 139.798399 104.548399) (width 0.2032) (layer F.Cu) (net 11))
 (segment (start 136.595189 99.353784) (end 136.595189 98.354811) (width 0.2032) (layer F.Cu) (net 11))
 (segment (start 139.798399 102.556993) (end 136.595189 99.353784) (width 0.2032) (layer F.Cu) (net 11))
 (segment (start 136.595189 98.354811) (end 137.377345 97.572655) (width 0.2032) (layer F.Cu) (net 11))
 (segment (start 137.377345 97.25243) (end 137.37902 97.250755) (width 0.2032) (layer F.Cu) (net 11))
 (segment (start 137.377345 97.572655) (end 137.377345 97.25243) (width 0.2032) (layer F.Cu) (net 11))
 (segment (start 137.37902 97.250755) (end 137.37902 89.61739) (width 0.2032) (layer F.Cu) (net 11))
 (segment (start 136.798399 89.036769) (end 136.798399 87.851601) (width 0.2032) (layer F.Cu) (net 11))
 (segment (start 137.37902 89.61739) (end 136.798399 89.036769) (width 0.2032) (layer F.Cu) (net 11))
 (via (at 136.8 87.85) (size 0.8) (drill 0.4) (layers F.Cu B.Cu) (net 11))
 (segment (start 136.798399 87.851601) (end 136.8 87.85) (width 0.2032) (layer F.Cu) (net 11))
 (segment (start 131.75 87.85) (end 131.726601 87.873399) (width 0.2032) (layer B.Cu) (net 11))
 (segment (start 136.8 87.85) (end 131.75 87.85) (width 0.2032) (layer B.Cu) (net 11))
 (segment (start 138.2 102.95) (end 138.41 103.16) (width 0.2032) (layer B.Cu) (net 12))
 (segment (start 138.41 103.16) (end 138.41 101.738819) (width 0.2032) (layer F.Cu) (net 12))
 (segment (start 138.41 101.738819) (end 136.191979 99.520799) (width 0.2032) (layer F.Cu) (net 12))
 (segment (start 136.191979 99.520799) (end 136.191979 98.187796) (width 0.2032) (layer F.Cu) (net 12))
 (segment (start 136.974135 97.085415) (end 136.97581 97.08374) (width 0.2032) (layer F.Cu) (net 12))
 (segment (start 136.974135 97.40564) (end 136.974135 97.085415) (width 0.2032) (layer F.Cu) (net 12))
 (segment (start 136.191979 98.187796) (end 136.974135 97.40564) (width 0.2032) (layer F.Cu) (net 12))
 (segment (start 136.97581 97.08374) (end 136.97581 89.784404) (width 0.2032) (layer F.Cu) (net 12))
 (segment (start 136.97581 89.784404) (end 136.39519 89.203784) (width 0.2032) (layer F.Cu) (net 12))
 (segment (start 136.39519 89.203784) (end 136.39519 88.48356) (width 0.2032) (layer F.Cu) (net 12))
 (via (at 136.737622 86.851945) (size 0.8) (drill 0.4) (layers F.Cu B.Cu) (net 12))
 (segment (start 136.098399 87.491168) (end 136.737622 86.851945) (width 0.2032) (layer F.Cu) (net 12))
 (segment (start 136.098399 88.186769) (end 136.098399 87.491168) (width 0.2032) (layer F.Cu) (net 12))
 (segment (start 136.39519 88.48356) (end 136.098399 88.186769) (width 0.2032) (layer F.Cu) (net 12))
 (segment (start 132.751945 86.851945) (end 132.75 86.85) (width 0.2032) (layer B.Cu) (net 12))
 (segment (start 136.737622 86.851945) (end 132.751945 86.851945) (width 0.2032) (layer B.Cu) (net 12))
 (segment (start 135.971174 86.199132) (end 135.971174 86.150345) (width 0.2032) (layer F.Cu) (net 13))
 (segment (start 135.764532 87.25481) (end 136.036021 86.983321) (width 0.2032) (layer F.Cu) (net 13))
 (segment (start 138.41 105.7) (end 137.258399 104.548399) (width 0.2032) (layer F.Cu) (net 13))
 (segment (start 137.258399 104.548399) (end 137.258399 101.157443) (width 0.2032) (layer F.Cu) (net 13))
 (segment (start 135.69519 87.25481) (end 135.764532 87.25481) (width 0.2032) (layer F.Cu) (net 13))
 (segment (start 135.991981 89.370799) (end 135.991981 88.650575) (width 0.2032) (layer F.Cu) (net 13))
 (segment (start 136.5726 96.916725) (end 136.5726 89.951418) (width 0.2032) (layer F.Cu) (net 13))
 (segment (start 136.5726 89.951418) (end 135.991981 89.370799) (width 0.2032) (layer F.Cu) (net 13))
 (segment (start 137.258399 101.157443) (end 135.636769 99.535813) (width 0.2032) (layer F.Cu) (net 13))
 (segment (start 135.636769 99.535813) (end 135.63677 98.172781) (width 0.2032) (layer F.Cu) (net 13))
 (segment (start 135.63677 98.172781) (end 136.570925 97.238626) (width 0.2032) (layer F.Cu) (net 13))
 (segment (start 135.69519 88.353784) (end 135.69519 87.25481) (width 0.2032) (layer F.Cu) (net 13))
 (segment (start 136.036021 86.983321) (end 136.036021 86.263979) (width 0.2032) (layer F.Cu) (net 13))
 (segment (start 136.570925 97.238626) (end 136.570925 96.9184) (width 0.2032) (layer F.Cu) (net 13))
 (via (at 135.971174 86.150345) (size 0.8) (drill 0.4) (layers F.Cu B.Cu) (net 13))
 (segment (start 136.570925 96.9184) (end 136.5726 96.916725) (width 0.2032) (layer F.Cu) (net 13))
 (segment (start 136.036021 86.263979) (end 135.971174 86.199132) (width 0.2032) (layer F.Cu) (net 13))
 (segment (start 135.991981 88.650575) (end 135.69519 88.353784) (width 0.2032) (layer F.Cu) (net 13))
 (segment (start 131.726601 85.873399) (end 130.75 86.85) (width 0.2032) (layer B.Cu) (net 13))
 (segment (start 135.694228 85.873399) (end 131.726601 85.873399) (width 0.2032) (layer B.Cu) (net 13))
 (segment (start 135.971174 86.150345) (end 135.694228 85.873399) (width 0.2032) (layer B.Cu) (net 13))
 (segment (start 135.87 103.16) (end 135.87 100.339268) (width 0.2032) (layer F.Cu) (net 14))
 (segment (start 135.87 100.339268) (end 135.23356 99.702827) (width 0.2032) (layer F.Cu) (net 14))
 (segment (start 135.23356 99.702827) (end 135.233561 98.005766) (width 0.2032) (layer F.Cu) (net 14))
 (segment (start 135.233561 98.005766) (end 136.167715 97.071612) (width 0.2032) (layer F.Cu) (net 14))
 (segment (start 136.15 96.73367) (end 136.15 90.099042) (width 0.2032) (layer F.Cu) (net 14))
 (segment (start 136.167715 96.751385) (end 136.15 96.73367) (width 0.2032) (layer F.Cu) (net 14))
 (segment (start 136.167715 97.071612) (end 136.167715 96.751385) (width 0.2032) (layer F.Cu) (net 14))
 (segment (start 136.15 90.099042) (end 135.588771 89.537814) (width 0.2032) (layer F.Cu) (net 14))
 (segment (start 135.588771 89.537814) (end 135.588771 88.817589) (width 0.2032) (layer F.Cu) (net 14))
 (via (at 136.1 84.85) (size 0.8) (drill 0.4) (layers F.Cu B.Cu) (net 14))
 (segment (start 135.269573 85.680427) (end 136.1 84.85) (width 0.2032) (layer F.Cu) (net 14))
 (segment (start 135.269573 88.498391) (end 135.269573 85.680427) (width 0.2032) (layer F.Cu) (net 14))
 (segment (start 135.588771 88.817589) (end 135.269573 88.498391) (width 0.2032) (layer F.Cu) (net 14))
 (segment (start 136.1 84.85) (end 132.75 84.85) (width 0.2032) (layer B.Cu) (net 14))
 (segment (start 134.718399 104.548399) (end 134.718399 102.681601) (width 0.2032) (layer F.Cu) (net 15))
 (segment (start 135.87 105.7) (end 134.718399 104.548399) (width 0.2032) (layer F.Cu) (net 15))
 (segment (start 134.718399 102.681601) (end 135.46679 101.93321) (width 0.2032) (layer F.Cu) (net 15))
 (segment (start 135.46679 100.506282) (end 134.830351 99.869842) (width 0.2032) (layer F.Cu) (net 15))
 (segment (start 135.46679 101.93321) (end 135.46679 100.506282) (width 0.2032) (layer F.Cu) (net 15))
 (segment (start 134.830351 99.869842) (end 134.830352 97.838751) (width 0.2032) (layer F.Cu) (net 15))
 (segment (start 135.757604 96.911499) (end 135.74679 96.900685) (width 0.2032) (layer F.Cu) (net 15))
 (segment (start 134.830352 97.838751) (end 135.757604 96.911499) (width 0.2032) (layer F.Cu) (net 15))
 (segment (start 135.74679 96.900685) (end 135.74679 90.6) (width 0.2032) (layer F.Cu) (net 15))
 (segment (start 135.74679 90.6) (end 135.74679 90.266057) (width 0.2032) (layer F.Cu) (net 15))
 (segment (start 135.74679 90.266057) (end 135.185561 89.704829) (width 0.2032) (layer F.Cu) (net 15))
 (segment (start 135.185561 89.704829) (end 135.185561 88.984603) (width 0.2032) (layer F.Cu) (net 15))
 (segment (start 135.185561 88.984603) (end 134.866364 88.665406) (width 0.2032) (layer F.Cu) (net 15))
 (segment (start 134.866364 88.665406) (end 134.866364 84.983636) (width 0.2032) (layer F.Cu) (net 15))
 (via (at 135.767179 83.907008) (size 0.8) (drill 0.4) (layers F.Cu B.Cu) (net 15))
 (segment (start 135.767179 84.082821) (end 135.767179 83.907008) (width 0.2032) (layer F.Cu) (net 15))
 (segment (start 134.866364 84.983636) (end 135.767179 84.082821) (width 0.2032) (layer F.Cu) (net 15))
 (segment (start 135.73357 83.873399) (end 135.767179 83.907008) (width 0.2032) (layer B.Cu) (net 15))
 (segment (start 131.726601 83.873399) (end 135.73357 83.873399) (width 0.2032) (layer B.Cu) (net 15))
 (segment (start 130.75 84.85) (end 131.726601 83.873399) (width 0.2032) (layer B.Cu) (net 15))
 (segment (start 135.3 90.625) (end 135.225 90.625) (width 0.2032) (layer B.Cu) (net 18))
 (via (at 134.05 90.6) (size 0.8) (drill 0.4) (layers F.Cu B.Cu) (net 18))
 (segment (start 134.05 76.85) (end 134.05 90.6) (width 0.2032) (layer F.Cu) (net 18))
 (segment (start 135.275 90.6) (end 135.3 90.625) (width 0.2032) (layer B.Cu) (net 18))
 (segment (start 134.05 90.6) (end 135.275 90.6) (width 0.2032) (layer B.Cu) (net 18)))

